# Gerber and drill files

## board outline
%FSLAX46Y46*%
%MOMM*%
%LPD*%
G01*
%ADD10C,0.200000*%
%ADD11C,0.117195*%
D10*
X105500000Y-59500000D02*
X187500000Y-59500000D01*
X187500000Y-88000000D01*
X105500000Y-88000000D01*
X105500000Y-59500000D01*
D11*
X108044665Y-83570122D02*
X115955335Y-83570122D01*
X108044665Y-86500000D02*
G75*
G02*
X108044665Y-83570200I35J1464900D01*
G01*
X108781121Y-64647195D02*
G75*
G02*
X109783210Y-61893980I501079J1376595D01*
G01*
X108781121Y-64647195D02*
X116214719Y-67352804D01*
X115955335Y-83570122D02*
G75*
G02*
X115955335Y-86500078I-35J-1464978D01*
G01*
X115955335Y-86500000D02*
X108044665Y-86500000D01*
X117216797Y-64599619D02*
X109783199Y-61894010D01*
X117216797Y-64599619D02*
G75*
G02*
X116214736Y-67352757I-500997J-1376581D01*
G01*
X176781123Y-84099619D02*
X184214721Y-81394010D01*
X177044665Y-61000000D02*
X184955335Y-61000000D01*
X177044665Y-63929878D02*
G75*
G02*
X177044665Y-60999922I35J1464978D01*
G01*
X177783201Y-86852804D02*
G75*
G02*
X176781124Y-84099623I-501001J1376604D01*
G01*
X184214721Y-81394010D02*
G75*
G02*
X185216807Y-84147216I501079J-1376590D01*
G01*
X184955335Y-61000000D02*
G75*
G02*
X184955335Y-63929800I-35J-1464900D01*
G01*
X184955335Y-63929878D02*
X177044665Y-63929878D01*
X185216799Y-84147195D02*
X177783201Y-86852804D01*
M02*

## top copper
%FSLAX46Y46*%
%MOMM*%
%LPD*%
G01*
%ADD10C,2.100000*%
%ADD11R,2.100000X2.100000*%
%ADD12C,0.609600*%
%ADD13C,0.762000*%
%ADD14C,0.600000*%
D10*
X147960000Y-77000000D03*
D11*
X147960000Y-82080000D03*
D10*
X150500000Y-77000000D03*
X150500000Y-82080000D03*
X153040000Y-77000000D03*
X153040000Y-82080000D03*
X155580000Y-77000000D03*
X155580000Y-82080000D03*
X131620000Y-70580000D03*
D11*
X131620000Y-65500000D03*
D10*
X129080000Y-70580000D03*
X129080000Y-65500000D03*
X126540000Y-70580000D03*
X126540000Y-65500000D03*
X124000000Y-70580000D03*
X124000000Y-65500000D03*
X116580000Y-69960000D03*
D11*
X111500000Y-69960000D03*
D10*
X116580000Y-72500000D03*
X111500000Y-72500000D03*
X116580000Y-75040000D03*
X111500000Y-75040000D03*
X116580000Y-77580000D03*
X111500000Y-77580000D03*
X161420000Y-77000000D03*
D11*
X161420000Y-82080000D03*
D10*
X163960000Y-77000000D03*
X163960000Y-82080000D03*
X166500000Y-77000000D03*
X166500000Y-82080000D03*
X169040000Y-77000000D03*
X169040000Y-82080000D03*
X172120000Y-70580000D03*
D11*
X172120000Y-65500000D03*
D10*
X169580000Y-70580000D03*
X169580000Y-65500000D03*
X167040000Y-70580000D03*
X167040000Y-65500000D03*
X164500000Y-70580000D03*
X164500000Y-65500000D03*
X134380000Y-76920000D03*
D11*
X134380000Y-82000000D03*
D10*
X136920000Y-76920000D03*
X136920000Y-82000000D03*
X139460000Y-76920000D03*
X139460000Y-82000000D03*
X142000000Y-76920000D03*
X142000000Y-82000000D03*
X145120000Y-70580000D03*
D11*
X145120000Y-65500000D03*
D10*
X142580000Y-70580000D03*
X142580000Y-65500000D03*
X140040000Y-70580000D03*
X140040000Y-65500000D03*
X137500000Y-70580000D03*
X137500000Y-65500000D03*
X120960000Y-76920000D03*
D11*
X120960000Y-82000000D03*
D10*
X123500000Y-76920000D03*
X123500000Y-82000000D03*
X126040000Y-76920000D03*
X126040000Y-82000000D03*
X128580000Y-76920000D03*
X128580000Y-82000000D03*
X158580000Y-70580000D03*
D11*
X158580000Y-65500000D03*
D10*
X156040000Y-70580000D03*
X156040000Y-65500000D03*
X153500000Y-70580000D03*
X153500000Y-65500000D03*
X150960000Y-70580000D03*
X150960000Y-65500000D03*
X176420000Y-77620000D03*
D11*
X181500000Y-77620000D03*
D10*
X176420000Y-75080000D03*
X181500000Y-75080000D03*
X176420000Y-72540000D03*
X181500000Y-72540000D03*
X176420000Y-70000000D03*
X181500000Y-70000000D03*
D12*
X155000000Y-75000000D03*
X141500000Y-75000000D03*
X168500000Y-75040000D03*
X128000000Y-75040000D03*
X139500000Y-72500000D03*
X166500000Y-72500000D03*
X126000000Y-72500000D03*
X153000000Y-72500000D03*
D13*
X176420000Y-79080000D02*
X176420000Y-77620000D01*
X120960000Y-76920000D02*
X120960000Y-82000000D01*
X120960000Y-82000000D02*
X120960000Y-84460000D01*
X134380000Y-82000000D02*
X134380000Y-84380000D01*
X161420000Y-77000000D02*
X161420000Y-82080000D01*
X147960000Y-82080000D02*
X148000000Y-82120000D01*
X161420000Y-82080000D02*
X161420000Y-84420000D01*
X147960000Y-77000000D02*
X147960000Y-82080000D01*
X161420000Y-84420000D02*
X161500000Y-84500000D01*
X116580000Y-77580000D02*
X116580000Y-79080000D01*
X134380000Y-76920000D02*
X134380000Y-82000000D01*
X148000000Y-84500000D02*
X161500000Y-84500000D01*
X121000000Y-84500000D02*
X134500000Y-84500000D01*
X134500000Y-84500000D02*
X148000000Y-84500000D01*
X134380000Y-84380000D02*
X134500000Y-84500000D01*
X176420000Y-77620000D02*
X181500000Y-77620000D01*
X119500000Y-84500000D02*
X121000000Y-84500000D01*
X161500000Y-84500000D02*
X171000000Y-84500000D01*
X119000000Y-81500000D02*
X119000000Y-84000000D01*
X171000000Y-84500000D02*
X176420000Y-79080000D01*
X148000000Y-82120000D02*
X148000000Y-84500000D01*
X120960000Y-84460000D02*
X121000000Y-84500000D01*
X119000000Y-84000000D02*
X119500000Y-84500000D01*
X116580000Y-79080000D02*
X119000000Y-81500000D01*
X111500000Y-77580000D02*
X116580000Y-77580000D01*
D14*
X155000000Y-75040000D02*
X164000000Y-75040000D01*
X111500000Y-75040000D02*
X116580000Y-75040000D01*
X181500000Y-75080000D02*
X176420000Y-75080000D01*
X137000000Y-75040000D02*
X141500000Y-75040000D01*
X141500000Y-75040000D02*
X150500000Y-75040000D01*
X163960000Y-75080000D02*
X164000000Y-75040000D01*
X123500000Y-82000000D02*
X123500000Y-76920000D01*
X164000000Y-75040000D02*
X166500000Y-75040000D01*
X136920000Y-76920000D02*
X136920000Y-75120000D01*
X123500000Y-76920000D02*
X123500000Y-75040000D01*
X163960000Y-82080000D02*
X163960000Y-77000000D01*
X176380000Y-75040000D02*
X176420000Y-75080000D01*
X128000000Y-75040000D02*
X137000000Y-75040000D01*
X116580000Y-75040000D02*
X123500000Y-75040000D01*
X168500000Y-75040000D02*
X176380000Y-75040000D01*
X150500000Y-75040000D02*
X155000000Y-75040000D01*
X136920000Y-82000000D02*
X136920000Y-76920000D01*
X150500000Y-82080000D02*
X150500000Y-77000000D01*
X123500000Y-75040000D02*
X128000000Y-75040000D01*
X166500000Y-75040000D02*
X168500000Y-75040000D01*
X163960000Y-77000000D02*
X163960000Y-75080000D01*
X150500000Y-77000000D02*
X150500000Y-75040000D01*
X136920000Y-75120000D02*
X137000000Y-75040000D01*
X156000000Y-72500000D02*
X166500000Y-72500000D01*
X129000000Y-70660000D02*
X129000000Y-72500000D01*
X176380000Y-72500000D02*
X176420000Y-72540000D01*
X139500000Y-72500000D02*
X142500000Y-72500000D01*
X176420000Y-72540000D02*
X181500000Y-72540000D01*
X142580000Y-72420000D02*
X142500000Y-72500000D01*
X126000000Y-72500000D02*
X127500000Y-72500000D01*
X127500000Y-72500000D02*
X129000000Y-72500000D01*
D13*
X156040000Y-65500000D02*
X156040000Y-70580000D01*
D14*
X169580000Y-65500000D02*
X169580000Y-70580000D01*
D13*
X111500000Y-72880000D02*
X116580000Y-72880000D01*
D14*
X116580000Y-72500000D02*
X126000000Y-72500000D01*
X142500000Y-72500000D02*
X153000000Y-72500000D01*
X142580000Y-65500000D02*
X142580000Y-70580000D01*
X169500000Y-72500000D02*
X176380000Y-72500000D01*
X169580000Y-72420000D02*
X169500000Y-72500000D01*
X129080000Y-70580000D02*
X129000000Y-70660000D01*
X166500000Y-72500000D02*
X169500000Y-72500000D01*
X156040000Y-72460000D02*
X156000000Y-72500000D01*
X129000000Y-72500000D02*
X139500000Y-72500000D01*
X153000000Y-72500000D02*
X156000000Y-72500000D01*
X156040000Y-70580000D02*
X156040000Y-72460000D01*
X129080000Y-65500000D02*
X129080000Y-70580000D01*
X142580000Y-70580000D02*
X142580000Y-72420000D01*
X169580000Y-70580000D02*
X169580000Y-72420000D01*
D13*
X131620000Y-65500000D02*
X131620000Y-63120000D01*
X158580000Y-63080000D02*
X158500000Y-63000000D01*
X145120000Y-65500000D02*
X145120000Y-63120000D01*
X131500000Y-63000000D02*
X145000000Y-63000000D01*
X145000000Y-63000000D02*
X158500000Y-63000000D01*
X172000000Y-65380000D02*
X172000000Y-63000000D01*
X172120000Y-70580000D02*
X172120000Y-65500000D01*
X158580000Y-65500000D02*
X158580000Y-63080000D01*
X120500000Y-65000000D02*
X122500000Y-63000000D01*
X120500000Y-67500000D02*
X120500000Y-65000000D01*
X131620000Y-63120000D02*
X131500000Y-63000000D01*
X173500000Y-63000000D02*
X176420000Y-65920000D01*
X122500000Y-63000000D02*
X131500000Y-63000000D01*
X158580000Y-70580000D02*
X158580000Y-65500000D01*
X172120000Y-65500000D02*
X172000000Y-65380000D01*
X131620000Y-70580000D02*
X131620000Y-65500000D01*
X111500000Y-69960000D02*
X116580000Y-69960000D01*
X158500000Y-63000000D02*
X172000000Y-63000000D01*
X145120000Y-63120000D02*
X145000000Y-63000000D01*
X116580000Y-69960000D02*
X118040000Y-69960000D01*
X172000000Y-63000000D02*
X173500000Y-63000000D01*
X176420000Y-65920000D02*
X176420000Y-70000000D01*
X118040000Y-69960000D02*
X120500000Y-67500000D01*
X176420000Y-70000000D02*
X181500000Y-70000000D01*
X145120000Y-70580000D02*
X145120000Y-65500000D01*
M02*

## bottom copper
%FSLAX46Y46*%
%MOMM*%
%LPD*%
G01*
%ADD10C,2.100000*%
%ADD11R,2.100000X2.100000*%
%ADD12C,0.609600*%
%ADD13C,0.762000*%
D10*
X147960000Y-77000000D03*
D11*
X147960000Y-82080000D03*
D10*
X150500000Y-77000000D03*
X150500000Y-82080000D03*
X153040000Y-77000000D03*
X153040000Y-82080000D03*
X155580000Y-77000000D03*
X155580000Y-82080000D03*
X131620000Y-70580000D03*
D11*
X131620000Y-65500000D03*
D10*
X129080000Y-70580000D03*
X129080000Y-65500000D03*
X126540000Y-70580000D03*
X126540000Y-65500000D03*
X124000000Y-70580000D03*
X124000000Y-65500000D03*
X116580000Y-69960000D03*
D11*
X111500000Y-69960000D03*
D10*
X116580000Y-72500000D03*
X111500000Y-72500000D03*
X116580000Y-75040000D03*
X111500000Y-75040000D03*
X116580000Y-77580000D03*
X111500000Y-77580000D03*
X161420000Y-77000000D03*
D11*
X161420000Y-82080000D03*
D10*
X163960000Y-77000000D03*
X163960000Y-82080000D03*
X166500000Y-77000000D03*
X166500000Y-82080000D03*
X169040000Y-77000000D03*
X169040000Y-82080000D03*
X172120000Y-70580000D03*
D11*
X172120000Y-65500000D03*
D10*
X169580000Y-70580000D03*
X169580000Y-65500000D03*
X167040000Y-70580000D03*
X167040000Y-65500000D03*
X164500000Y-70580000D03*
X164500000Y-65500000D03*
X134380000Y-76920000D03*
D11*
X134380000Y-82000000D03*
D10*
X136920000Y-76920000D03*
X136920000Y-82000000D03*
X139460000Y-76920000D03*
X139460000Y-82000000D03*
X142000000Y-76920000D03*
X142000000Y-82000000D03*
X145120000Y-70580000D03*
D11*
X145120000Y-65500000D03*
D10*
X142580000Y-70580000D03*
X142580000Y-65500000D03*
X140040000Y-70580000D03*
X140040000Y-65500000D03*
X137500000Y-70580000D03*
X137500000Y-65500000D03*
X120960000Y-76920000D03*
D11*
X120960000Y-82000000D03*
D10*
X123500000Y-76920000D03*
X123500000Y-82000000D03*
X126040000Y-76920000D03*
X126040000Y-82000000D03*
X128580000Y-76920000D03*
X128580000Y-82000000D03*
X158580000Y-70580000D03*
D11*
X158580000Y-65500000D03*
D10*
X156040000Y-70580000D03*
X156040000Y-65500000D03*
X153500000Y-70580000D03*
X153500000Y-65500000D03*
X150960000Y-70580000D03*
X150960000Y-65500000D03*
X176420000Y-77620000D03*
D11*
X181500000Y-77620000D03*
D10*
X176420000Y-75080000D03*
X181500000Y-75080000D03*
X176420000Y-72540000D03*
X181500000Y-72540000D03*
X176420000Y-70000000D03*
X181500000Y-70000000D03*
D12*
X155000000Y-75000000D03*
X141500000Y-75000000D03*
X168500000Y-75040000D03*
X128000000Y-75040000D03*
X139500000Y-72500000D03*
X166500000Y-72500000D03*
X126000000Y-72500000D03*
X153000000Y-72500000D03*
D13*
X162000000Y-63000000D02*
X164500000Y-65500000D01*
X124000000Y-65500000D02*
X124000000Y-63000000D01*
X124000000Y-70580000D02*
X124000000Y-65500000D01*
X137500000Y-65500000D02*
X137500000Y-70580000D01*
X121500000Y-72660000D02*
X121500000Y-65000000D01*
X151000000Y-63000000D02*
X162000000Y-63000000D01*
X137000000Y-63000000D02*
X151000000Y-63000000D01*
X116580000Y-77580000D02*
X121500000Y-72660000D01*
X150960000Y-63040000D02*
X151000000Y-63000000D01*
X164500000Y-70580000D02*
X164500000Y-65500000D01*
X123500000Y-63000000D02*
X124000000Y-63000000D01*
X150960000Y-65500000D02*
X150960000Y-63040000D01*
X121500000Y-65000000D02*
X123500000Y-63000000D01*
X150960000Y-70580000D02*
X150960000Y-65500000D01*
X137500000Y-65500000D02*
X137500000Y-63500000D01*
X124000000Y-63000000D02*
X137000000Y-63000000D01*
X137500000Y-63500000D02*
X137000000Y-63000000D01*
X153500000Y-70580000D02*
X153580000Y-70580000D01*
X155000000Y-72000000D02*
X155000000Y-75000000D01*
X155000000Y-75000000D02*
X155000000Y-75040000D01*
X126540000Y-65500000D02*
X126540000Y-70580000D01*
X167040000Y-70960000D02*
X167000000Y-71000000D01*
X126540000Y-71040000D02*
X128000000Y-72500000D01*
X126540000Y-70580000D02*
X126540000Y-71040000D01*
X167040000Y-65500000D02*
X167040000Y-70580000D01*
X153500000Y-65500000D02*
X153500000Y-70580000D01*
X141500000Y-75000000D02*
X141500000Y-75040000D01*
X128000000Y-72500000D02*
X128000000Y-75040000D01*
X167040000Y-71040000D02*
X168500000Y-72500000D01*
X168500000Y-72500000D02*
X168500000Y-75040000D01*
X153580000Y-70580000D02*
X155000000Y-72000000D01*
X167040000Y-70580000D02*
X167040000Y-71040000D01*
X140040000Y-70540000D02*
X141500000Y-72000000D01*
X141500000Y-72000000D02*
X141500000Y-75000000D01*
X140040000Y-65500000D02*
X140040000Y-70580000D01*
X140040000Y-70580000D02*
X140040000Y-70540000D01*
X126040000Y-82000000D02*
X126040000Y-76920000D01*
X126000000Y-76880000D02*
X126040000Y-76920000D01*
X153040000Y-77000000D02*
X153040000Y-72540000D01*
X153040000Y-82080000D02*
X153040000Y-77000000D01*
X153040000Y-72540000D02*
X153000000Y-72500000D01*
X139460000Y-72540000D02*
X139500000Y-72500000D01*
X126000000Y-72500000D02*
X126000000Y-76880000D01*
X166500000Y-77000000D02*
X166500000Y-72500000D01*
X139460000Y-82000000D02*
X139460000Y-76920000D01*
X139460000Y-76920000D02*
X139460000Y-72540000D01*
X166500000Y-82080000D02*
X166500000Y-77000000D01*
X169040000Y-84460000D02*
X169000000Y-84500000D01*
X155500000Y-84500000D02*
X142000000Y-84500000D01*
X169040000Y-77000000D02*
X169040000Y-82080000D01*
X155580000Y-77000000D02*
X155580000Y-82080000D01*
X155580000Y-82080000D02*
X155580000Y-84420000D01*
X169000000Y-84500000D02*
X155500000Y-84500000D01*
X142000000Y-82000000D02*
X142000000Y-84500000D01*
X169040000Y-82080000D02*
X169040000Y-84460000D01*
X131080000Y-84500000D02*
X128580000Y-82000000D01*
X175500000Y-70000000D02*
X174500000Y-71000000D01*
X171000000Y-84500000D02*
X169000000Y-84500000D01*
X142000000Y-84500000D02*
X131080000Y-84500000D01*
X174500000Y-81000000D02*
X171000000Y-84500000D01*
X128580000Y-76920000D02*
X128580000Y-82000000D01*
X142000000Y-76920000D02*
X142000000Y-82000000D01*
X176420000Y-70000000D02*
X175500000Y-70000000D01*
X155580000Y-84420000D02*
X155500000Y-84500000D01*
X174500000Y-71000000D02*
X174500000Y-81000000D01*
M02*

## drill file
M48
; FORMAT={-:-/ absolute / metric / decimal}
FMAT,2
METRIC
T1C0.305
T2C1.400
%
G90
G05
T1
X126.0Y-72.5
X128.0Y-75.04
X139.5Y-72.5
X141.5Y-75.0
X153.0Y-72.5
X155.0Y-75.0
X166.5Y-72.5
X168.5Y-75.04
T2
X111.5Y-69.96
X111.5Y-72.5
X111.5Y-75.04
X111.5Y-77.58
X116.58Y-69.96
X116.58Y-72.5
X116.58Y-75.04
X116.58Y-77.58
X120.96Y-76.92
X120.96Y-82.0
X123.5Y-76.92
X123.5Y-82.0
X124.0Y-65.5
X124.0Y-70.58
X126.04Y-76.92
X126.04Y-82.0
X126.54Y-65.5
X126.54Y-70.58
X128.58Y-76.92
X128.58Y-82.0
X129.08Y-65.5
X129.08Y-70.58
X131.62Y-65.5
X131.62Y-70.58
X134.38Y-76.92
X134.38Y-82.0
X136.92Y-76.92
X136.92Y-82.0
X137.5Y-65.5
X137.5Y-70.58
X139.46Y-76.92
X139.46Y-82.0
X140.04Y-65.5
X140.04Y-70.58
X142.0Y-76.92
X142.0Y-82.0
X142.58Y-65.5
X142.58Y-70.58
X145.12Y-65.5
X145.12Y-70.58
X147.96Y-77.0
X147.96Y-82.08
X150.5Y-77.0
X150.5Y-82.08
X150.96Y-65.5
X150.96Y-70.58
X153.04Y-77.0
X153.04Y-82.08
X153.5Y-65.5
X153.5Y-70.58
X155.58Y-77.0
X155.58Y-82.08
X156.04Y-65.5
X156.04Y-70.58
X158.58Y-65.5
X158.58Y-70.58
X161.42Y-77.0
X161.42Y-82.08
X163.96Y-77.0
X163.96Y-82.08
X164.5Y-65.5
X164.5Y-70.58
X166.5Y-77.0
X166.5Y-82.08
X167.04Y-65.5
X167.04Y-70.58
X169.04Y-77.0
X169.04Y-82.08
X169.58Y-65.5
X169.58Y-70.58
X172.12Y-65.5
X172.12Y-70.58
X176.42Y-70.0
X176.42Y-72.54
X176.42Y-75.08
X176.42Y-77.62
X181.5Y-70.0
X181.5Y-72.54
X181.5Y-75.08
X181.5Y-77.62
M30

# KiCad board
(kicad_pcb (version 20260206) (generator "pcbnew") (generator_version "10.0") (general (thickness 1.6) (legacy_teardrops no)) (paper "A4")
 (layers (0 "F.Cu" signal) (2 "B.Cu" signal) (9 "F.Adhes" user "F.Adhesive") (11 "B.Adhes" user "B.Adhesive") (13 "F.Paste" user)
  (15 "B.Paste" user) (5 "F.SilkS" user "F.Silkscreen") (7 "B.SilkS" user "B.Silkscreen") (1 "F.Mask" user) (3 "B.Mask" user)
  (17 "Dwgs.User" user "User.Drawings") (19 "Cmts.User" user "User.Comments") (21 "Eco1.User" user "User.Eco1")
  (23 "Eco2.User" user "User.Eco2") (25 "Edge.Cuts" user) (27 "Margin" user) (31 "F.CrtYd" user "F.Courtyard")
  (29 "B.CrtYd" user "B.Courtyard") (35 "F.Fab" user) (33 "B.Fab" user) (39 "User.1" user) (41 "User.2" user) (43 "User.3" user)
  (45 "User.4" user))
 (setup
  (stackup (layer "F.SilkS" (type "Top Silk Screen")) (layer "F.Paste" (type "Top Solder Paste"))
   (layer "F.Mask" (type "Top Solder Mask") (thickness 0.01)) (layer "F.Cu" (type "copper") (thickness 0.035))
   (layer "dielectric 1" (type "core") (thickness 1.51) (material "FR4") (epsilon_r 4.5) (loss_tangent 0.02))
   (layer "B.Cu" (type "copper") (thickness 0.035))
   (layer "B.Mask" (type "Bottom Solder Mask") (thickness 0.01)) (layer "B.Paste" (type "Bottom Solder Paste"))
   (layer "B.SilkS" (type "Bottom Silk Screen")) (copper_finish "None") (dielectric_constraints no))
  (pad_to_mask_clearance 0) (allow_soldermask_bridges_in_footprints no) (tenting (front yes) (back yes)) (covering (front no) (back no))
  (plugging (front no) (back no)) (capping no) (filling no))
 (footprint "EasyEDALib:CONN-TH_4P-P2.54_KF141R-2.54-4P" (layer "F.Cu") (at 151.77 79.54)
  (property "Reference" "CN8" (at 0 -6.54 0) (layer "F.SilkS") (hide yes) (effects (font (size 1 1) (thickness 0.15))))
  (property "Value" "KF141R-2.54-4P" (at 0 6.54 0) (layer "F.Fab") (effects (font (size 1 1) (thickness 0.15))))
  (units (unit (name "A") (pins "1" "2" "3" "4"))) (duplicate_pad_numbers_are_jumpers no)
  (pad "1" thru_hole circle (at -3.81 -2.54 180) (size 2.1 2.1) (drill 1.399998) (layers "*.Cu" "*.Mask") (remove_unused_layers no)
   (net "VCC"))
  (pad "1" thru_hole rect (at -3.81 2.54 180) (size 2.1 2.1) (drill 1.399998) (layers "*.Cu" "*.Mask") (remove_unused_layers no) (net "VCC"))
  (pad "2" thru_hole circle (at -1.27 -2.54 180) (size 2.1 2.1) (drill 1.399998) (layers "*.Cu" "*.Mask") (remove_unused_layers no)
   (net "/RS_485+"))
  (pad "2" thru_hole circle (at -1.27 2.54 180) (size 2.1 2.1) (drill 1.399998) (layers "*.Cu" "*.Mask") (remove_unused_layers no)
   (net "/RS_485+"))
  (pad "3" thru_hole circle (at 1.27 -2.54 180) (size 2.1 2.1) (drill 1.399998) (layers "*.Cu" "*.Mask") (remove_unused_layers no)
   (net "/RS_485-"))
  (pad "3" thru_hole circle (at 1.27 2.54 180) (size 2.1 2.1) (drill 1.399998) (layers "*.Cu" "*.Mask") (remove_unused_layers no)
   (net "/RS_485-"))
  (pad "4" thru_hole circle (at 3.81 -2.54 180) (size 2.1 2.1) (drill 1.399998) (layers "*.Cu" "*.Mask") (remove_unused_layers no)
   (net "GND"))
  (pad "4" thru_hole circle (at 3.81 2.54 180) (size 2.1 2.1) (drill 1.399998) (layers "*.Cu" "*.Mask") (remove_unused_layers no)
   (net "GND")))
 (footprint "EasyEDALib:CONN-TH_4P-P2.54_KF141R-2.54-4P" (layer "F.Cu") (at 127.81 68.04 180)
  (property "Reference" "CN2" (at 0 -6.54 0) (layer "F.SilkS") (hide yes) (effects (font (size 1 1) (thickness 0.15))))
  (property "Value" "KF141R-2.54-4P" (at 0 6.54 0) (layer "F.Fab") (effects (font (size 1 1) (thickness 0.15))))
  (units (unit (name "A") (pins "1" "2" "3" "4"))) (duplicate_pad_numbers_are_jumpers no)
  (pad "1" thru_hole circle (at -3.81 -2.54) (size 2.1 2.1) (drill 1.399998) (layers "*.Cu" "*.Mask") (remove_unused_layers no) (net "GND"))
  (pad "1" thru_hole rect (at -3.81 2.54) (size 2.1 2.1) (drill 1.399998) (layers "*.Cu" "*.Mask") (remove_unused_layers no) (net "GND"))
  (pad "2" thru_hole circle (at -1.27 -2.54) (size 2.1 2.1) (drill 1.399998) (layers "*.Cu" "*.Mask") (remove_unused_layers no)
   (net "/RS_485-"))
  (pad "2" thru_hole circle (at -1.27 2.54) (size 2.1 2.1) (drill 1.399998) (layers "*.Cu" "*.Mask") (remove_unused_layers no)
   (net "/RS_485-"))
  (pad "3" thru_hole circle (at 1.27 -2.54) (size 2.1 2.1) (drill 1.399998) (layers "*.Cu" "*.Mask") (remove_unused_layers no)
   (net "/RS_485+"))
  (pad "3" thru_hole circle (at 1.27 2.54) (size 2.1 2.1) (drill 1.399998) (layers "*.Cu" "*.Mask") (remove_unused_layers no)
   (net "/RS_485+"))
  (pad "4" thru_hole circle (at 3.81 -2.54) (size 2.1 2.1) (drill 1.399998) (layers "*.Cu" "*.Mask") (remove_unused_layers no) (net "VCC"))
  (pad "4" thru_hole circle (at 3.81 2.54) (size 2.1 2.1) (drill 1.399998) (layers "*.Cu" "*.Mask") (remove_unused_layers no) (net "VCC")))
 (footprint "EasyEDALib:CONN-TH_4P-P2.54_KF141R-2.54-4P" (layer "F.Cu") (at 114.04 73.77 -90)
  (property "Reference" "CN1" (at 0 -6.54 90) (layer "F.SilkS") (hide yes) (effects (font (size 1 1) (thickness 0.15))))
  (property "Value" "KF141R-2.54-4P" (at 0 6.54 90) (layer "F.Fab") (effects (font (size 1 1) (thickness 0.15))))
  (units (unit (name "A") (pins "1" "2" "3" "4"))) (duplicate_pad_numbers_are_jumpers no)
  (pad "1" thru_hole circle (at -3.81 -2.54 90) (size 2.1 2.1) (drill 1.399998) (layers "*.Cu" "*.Mask") (remove_unused_layers no)
   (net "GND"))
  (pad "1" thru_hole rect (at -3.81 2.54 90) (size 2.1 2.1) (drill 1.399998) (layers "*.Cu" "*.Mask") (remove_unused_layers no) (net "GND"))
  (pad "2" thru_hole circle (at -1.27 -2.54 90) (size 2.1 2.1) (drill 1.399998) (layers "*.Cu" "*.Mask") (remove_unused_layers no)
   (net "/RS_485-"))
  (pad "2" thru_hole circle (at -1.27 2.54 90) (size 2.1 2.1) (drill 1.399998) (layers "*.Cu" "*.Mask") (remove_unused_layers no)
   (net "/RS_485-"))
  (pad "3" thru_hole circle (at 1.27 -2.54 90) (size 2.1 2.1) (drill 1.399998) (layers "*.Cu" "*.Mask") (remove_unused_layers no)
   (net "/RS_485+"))
  (pad "3" thru_hole circle (at 1.27 2.54 90) (size 2.1 2.1) (drill 1.399998) (layers "*.Cu" "*.Mask") (remove_unused_layers no)
   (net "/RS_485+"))
  (pad "4" thru_hole circle (at 3.81 -2.54 90) (size 2.1 2.1) (drill 1.399998) (layers "*.Cu" "*.Mask") (remove_unused_layers no)
   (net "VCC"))
  (pad "4" thru_hole circle (at 3.81 2.54 90) (size 2.1 2.1) (drill 1.399998) (layers "*.Cu" "*.Mask") (remove_unused_layers no) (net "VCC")))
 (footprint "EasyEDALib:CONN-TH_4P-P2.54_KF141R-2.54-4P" (layer "F.Cu") (at 165.23 79.54)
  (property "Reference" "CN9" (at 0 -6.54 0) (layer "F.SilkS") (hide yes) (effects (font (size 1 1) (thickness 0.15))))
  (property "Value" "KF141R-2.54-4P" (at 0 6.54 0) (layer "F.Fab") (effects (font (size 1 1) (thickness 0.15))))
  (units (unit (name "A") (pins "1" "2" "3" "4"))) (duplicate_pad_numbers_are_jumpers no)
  (pad "1" thru_hole circle (at -3.81 -2.54 180) (size 2.1 2.1) (drill 1.399998) (layers "*.Cu" "*.Mask") (remove_unused_layers no)
   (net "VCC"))
  (pad "1" thru_hole rect (at -3.81 2.54 180) (size 2.1 2.1) (drill 1.399998) (layers "*.Cu" "*.Mask") (remove_unused_layers no) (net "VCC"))
  (pad "2" thru_hole circle (at -1.27 -2.54 180) (size 2.1 2.1) (drill 1.399998) (layers "*.Cu" "*.Mask") (remove_unused_layers no)
   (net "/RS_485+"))
  (pad "2" thru_hole circle (at -1.27 2.54 180) (size 2.1 2.1) (drill 1.399998) (layers "*.Cu" "*.Mask") (remove_unused_layers no)
   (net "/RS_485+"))
  (pad "3" thru_hole circle (at 1.27 -2.54 180) (size 2.1 2.1) (drill 1.399998) (layers "*.Cu" "*.Mask") (remove_unused_layers no)
   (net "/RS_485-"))
  (pad "3" thru_hole circle (at 1.27 2.54 180) (size 2.1 2.1) (drill 1.399998) (layers "*.Cu" "*.Mask") (remove_unused_layers no)
   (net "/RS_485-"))
  (pad "4" thru_hole circle (at 3.81 -2.54 180) (size 2.1 2.1) (drill 1.399998) (layers "*.Cu" "*.Mask") (remove_unused_layers no)
   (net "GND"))
  (pad "4" thru_hole circle (at 3.81 2.54 180) (size 2.1 2.1) (drill 1.399998) (layers "*.Cu" "*.Mask") (remove_unused_layers no)
   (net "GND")))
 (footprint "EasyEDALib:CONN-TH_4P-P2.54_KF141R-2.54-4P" (layer "F.Cu") (at 168.31 68.04 180)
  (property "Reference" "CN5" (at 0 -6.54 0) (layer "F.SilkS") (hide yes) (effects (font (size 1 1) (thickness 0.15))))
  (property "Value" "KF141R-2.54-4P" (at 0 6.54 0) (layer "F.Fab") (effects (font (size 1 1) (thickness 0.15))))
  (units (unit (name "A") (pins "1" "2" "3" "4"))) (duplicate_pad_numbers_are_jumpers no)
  (pad "1" thru_hole circle (at -3.81 -2.54) (size 2.1 2.1) (drill 1.399998) (layers "*.Cu" "*.Mask") (remove_unused_layers no) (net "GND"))
  (pad "1" thru_hole rect (at -3.81 2.54) (size 2.1 2.1) (drill 1.399998) (layers "*.Cu" "*.Mask") (remove_unused_layers no) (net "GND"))
  (pad "2" thru_hole circle (at -1.27 -2.54) (size 2.1 2.1) (drill 1.399998) (layers "*.Cu" "*.Mask") (remove_unused_layers no)
   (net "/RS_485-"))
  (pad "2" thru_hole circle (at -1.27 2.54) (size 2.1 2.1) (drill 1.399998) (layers "*.Cu" "*.Mask") (remove_unused_layers no)
   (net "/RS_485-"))
  (pad "3" thru_hole circle (at 1.27 -2.54) (size 2.1 2.1) (drill 1.399998) (layers "*.Cu" "*.Mask") (remove_unused_layers no)
   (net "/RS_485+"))
  (pad "3" thru_hole circle (at 1.27 2.54) (size 2.1 2.1) (drill 1.399998) (layers "*.Cu" "*.Mask") (remove_unused_layers no)
   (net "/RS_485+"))
  (pad "4" thru_hole circle (at 3.81 -2.54) (size 2.1 2.1) (drill 1.399998) (layers "*.Cu" "*.Mask") (remove_unused_layers no) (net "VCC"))
  (pad "4" thru_hole circle (at 3.81 2.54) (size 2.1 2.1) (drill 1.399998) (layers "*.Cu" "*.Mask") (remove_unused_layers no) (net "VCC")))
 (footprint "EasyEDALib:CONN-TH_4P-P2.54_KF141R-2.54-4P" (layer "F.Cu") (at 138.19 79.46)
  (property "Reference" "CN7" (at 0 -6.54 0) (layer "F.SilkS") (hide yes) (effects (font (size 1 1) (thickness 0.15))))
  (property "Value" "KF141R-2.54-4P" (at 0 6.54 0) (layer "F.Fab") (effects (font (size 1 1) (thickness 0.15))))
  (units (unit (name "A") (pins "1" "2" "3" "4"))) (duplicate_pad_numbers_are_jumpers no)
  (pad "1" thru_hole circle (at -3.81 -2.54 180) (size 2.1 2.1) (drill 1.399998) (layers "*.Cu" "*.Mask") (remove_unused_layers no)
   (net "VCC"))
  (pad "1" thru_hole rect (at -3.81 2.54 180) (size 2.1 2.1) (drill 1.399998) (layers "*.Cu" "*.Mask") (remove_unused_layers no) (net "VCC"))
  (pad "2" thru_hole circle (at -1.27 -2.54 180) (size 2.1 2.1) (drill 1.399998) (layers "*.Cu" "*.Mask") (remove_unused_layers no)
   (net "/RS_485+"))
  (pad "2" thru_hole circle (at -1.27 2.54 180) (size 2.1 2.1) (drill 1.399998) (layers "*.Cu" "*.Mask") (remove_unused_layers no)
   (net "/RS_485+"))
  (pad "3" thru_hole circle (at 1.27 -2.54 180) (size 2.1 2.1) (drill 1.399998) (layers "*.Cu" "*.Mask") (remove_unused_layers no)
   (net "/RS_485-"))
  (pad "3" thru_hole circle (at 1.27 2.54 180) (size 2.1 2.1) (drill 1.399998) (layers "*.Cu" "*.Mask") (remove_unused_layers no)
   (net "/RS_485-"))
  (pad "4" thru_hole circle (at 3.81 -2.54 180) (size 2.1 2.1) (drill 1.399998) (layers "*.Cu" "*.Mask") (remove_unused_layers no)
   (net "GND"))
  (pad "4" thru_hole circle (at 3.81 2.54 180) (size 2.1 2.1) (drill 1.399998) (layers "*.Cu" "*.Mask") (remove_unused_layers no)
   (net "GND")))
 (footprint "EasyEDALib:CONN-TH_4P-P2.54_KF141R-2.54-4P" (layer "F.Cu") (at 141.31 68.04 180)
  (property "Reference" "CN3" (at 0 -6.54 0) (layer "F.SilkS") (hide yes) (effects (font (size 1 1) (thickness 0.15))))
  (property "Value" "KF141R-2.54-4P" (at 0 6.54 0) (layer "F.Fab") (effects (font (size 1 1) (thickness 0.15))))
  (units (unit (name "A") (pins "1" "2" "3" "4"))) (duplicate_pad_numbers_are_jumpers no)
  (pad "1" thru_hole circle (at -3.81 -2.54) (size 2.1 2.1) (drill 1.399998) (layers "*.Cu" "*.Mask") (remove_unused_layers no) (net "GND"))
  (pad "1" thru_hole rect (at -3.81 2.54) (size 2.1 2.1) (drill 1.399998) (layers "*.Cu" "*.Mask") (remove_unused_layers no) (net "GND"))
  (pad "2" thru_hole circle (at -1.27 -2.54) (size 2.1 2.1) (drill 1.399998) (layers "*.Cu" "*.Mask") (remove_unused_layers no)
   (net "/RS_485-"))
  (pad "2" thru_hole circle (at -1.27 2.54) (size 2.1 2.1) (drill 1.399998) (layers "*.Cu" "*.Mask") (remove_unused_layers no)
   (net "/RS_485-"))
  (pad "3" thru_hole circle (at 1.27 -2.54) (size 2.1 2.1) (drill 1.399998) (layers "*.Cu" "*.Mask") (remove_unused_layers no)
   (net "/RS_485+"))
  (pad "3" thru_hole circle (at 1.27 2.54) (size 2.1 2.1) (drill 1.399998) (layers "*.Cu" "*.Mask") (remove_unused_layers no)
   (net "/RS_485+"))
  (pad "4" thru_hole circle (at 3.81 -2.54) (size 2.1 2.1) (drill 1.399998) (layers "*.Cu" "*.Mask") (remove_unused_layers no) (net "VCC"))
  (pad "4" thru_hole circle (at 3.81 2.54) (size 2.1 2.1) (drill 1.399998) (layers "*.Cu" "*.Mask") (remove_unused_layers no) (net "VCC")))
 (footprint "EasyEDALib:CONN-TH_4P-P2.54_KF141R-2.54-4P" (layer "F.Cu") (at 124.77 79.46)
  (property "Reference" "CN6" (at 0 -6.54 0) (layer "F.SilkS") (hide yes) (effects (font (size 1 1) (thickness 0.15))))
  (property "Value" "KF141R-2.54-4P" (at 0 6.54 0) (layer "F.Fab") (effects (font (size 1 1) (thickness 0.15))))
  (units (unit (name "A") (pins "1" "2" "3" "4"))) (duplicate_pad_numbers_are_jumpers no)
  (pad "1" thru_hole circle (at -3.81 -2.54 180) (size 2.1 2.1) (drill 1.399998) (layers "*.Cu" "*.Mask") (remove_unused_layers no)
   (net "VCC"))
  (pad "1" thru_hole rect (at -3.81 2.54 180) (size 2.1 2.1) (drill 1.399998) (layers "*.Cu" "*.Mask") (remove_unused_layers no) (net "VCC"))
  (pad "2" thru_hole circle (at -1.27 -2.54 180) (size 2.1 2.1) (drill 1.399998) (layers "*.Cu" "*.Mask") (remove_unused_layers no)
   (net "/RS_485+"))
  (pad "2" thru_hole circle (at -1.27 2.54 180) (size 2.1 2.1) (drill 1.399998) (layers "*.Cu" "*.Mask") (remove_unused_layers no)
   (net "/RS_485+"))
  (pad "3" thru_hole circle (at 1.27 -2.54 180) (size 2.1 2.1) (drill 1.399998) (layers "*.Cu" "*.Mask") (remove_unused_layers no)
   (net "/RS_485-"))
  (pad "3" thru_hole circle (at 1.27 2.54 180) (size 2.1 2.1) (drill 1.399998) (layers "*.Cu" "*.Mask") (remove_unused_layers no)
   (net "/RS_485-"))
  (pad "4" thru_hole circle (at 3.81 -2.54 180) (size 2.1 2.1) (drill 1.399998) (layers "*.Cu" "*.Mask") (remove_unused_layers no)
   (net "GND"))
  (pad "4" thru_hole circle (at 3.81 2.54 180) (size 2.1 2.1) (drill 1.399998) (layers "*.Cu" "*.Mask") (remove_unused_layers no)
   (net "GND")))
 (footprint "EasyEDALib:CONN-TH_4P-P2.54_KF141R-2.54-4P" (layer "F.Cu") (at 154.77 68.04 180)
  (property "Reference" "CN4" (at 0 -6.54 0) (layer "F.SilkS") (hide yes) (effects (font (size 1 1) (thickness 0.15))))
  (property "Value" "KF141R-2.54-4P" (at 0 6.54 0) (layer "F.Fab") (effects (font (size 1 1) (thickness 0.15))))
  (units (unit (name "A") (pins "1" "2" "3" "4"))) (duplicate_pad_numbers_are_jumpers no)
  (pad "1" thru_hole circle (at -3.81 -2.54) (size 2.1 2.1) (drill 1.399998) (layers "*.Cu" "*.Mask") (remove_unused_layers no) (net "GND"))
  (pad "1" thru_hole rect (at -3.81 2.54) (size 2.1 2.1) (drill 1.399998) (layers "*.Cu" "*.Mask") (remove_unused_layers no) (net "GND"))
  (pad "2" thru_hole circle (at -1.27 -2.54) (size 2.1 2.1) (drill 1.399998) (layers "*.Cu" "*.Mask") (remove_unused_layers no)
   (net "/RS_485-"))
  (pad "2" thru_hole circle (at -1.27 2.54) (size 2.1 2.1) (drill 1.399998) (layers "*.Cu" "*.Mask") (remove_unused_layers no)
   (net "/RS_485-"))
  (pad "3" thru_hole circle (at 1.27 -2.54) (size 2.1 2.1) (drill 1.399998) (layers "*.Cu" "*.Mask") (remove_unused_layers no)
   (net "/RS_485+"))
  (pad "3" thru_hole circle (at 1.27 2.54) (size 2.1 2.1) (drill 1.399998) (layers "*.Cu" "*.Mask") (remove_unused_layers no)
   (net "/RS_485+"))
  (pad "4" thru_hole circle (at 3.81 -2.54) (size 2.1 2.1) (drill 1.399998) (layers "*.Cu" "*.Mask") (remove_unused_layers no) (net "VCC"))
  (pad "4" thru_hole circle (at 3.81 2.54) (size 2.1 2.1) (drill 1.399998) (layers "*.Cu" "*.Mask") (remove_unused_layers no) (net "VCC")))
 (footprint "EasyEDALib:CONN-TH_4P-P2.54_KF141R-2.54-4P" (layer "F.Cu") (at 178.96 73.81 90)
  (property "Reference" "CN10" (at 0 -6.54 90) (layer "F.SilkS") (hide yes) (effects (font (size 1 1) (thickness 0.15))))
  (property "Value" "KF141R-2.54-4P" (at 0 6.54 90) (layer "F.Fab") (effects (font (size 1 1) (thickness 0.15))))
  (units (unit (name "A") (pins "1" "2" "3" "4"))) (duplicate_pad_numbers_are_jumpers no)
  (pad "1" thru_hole circle (at -3.81 -2.54 270) (size 2.1 2.1) (drill 1.399998) (layers "*.Cu" "*.Mask") (remove_unused_layers no)
   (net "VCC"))
  (pad "1" thru_hole rect (at -3.81 2.54 270) (size 2.1 2.1) (drill 1.399998) (layers "*.Cu" "*.Mask") (remove_unused_layers no) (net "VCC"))
  (pad "2" thru_hole circle (at -1.27 -2.54 270) (size 2.1 2.1) (drill 1.399998) (layers "*.Cu" "*.Mask") (remove_unused_layers no)
   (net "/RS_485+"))
  (pad "2" thru_hole circle (at -1.27 2.54 270) (size 2.1 2.1) (drill 1.399998) (layers "*.Cu" "*.Mask") (remove_unused_layers no)
   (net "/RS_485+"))
  (pad "3" thru_hole circle (at 1.27 -2.54 270) (size 2.1 2.1) (drill 1.399998) (layers "*.Cu" "*.Mask") (remove_unused_layers no)
   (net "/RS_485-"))
  (pad "3" thru_hole circle (at 1.27 2.54 270) (size 2.1 2.1) (drill 1.399998) (layers "*.Cu" "*.Mask") (remove_unused_layers no)
   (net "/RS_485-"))
  (pad "4" thru_hole circle (at 3.81 -2.54 270) (size 2.1 2.1) (drill 1.399998) (layers "*.Cu" "*.Mask") (remove_unused_layers no)
   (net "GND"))
  (pad "4" thru_hole circle (at 3.81 2.54 270) (size 2.1 2.1) (drill 1.399998) (layers "*.Cu" "*.Mask") (remove_unused_layers no)
   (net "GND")))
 (gr_rect (start 105.5 59.5) (end 187.5 88) (stroke (width 0.2) (type solid)) (fill no) (layer "Edge.Cuts"))
 (gr_line (start 108.044665 83.570122) (end 115.955335 83.570122) (stroke (width 0.117195) (type default)) (layer "Edge.Cuts"))
 (gr_arc (start 108.044665 86.5) (mid 106.579726 85.035061) (end 108.044665 83.570122) (stroke (width 0.117195) (type default))
  (layer "Edge.Cuts"))
 (gr_arc (start 108.781121 64.647195) (mid 107.905565 62.76956) (end 109.783199 61.89401) (stroke (width 0.117195) (type default))
  (layer "Edge.Cuts"))
 (gr_line (start 108.781121 64.647195) (end 116.214719 67.352804) (stroke (width 0.117195) (type default)) (layer "Edge.Cuts"))
 (gr_arc (start 115.955335 83.570122) (mid 117.420274 85.035061) (end 115.955335 86.5) (stroke (width 0.117195) (type default))
  (layer "Edge.Cuts"))
 (gr_line (start 115.955335 86.5) (end 108.044665 86.5) (stroke (width 0.117195) (type default)) (layer "Edge.Cuts"))
 (gr_line (start 117.216797 64.599619) (end 109.783199 61.89401) (stroke (width 0.117195) (type default)) (layer "Edge.Cuts"))
 (gr_arc (start 117.216797 64.599619) (mid 118.092351 66.477251) (end 116.214719 67.352804) (stroke (width 0.117195) (type default))
  (layer "Edge.Cuts"))
 (gr_line (start 176.781123 84.099619) (end 184.214721 81.39401) (stroke (width 0.117195) (type default)) (layer "Edge.Cuts"))
 (gr_line (start 177.044665 61) (end 184.955335 61) (stroke (width 0.117195) (type default)) (layer "Edge.Cuts"))
 (gr_arc (start 177.044665 63.929878) (mid 175.579726 62.464939) (end 177.044665 61) (stroke (width 0.117195) (type default))
  (layer "Edge.Cuts"))
 (gr_arc (start 177.783201 86.852804) (mid 175.905569 85.97725) (end 176.781123 84.099619) (stroke (width 0.117195) (type default))
  (layer "Edge.Cuts"))
 (gr_arc (start 184.214721 81.39401) (mid 186.092353 82.269564) (end 185.216799 84.147195) (stroke (width 0.117195) (type default))
  (layer "Edge.Cuts"))
 (gr_arc (start 184.955335 61) (mid 186.420274 62.464939) (end 184.955335 63.929878) (stroke (width 0.117195) (type default))
  (layer "Edge.Cuts"))
 (gr_line (start 184.955335 63.929878) (end 177.044665 63.929878) (stroke (width 0.117195) (type default)) (layer "Edge.Cuts"))
 (gr_line (start 185.216799 84.147195) (end 177.783201 86.852804) (stroke (width 0.117195) (type default)) (layer "Edge.Cuts"))
 (segment (start 176.42 79.08) (end 176.42 77.62) (width 0.762) (layer "F.Cu") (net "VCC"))
 (segment (start 120.96 76.92) (end 120.96 82) (width 0.762) (layer "F.Cu") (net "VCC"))
 (segment (start 120.96 82) (end 120.96 84.46) (width 0.762) (layer "F.Cu") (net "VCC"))
 (segment (start 134.38 82) (end 134.38 84.38) (width 0.762) (layer "F.Cu") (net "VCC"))
 (segment (start 161.42 77) (end 161.42 82.08) (width 0.762) (layer "F.Cu") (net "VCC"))
 (segment (start 147.96 82.08) (end 148 82.12) (width 0.762) (layer "F.Cu") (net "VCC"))
 (segment (start 161.42 82.08) (end 161.42 84.42) (width 0.762) (layer "F.Cu") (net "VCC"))
 (segment (start 147.96 77) (end 147.96 82.08) (width 0.762) (layer "F.Cu") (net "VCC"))
 (segment (start 161.42 84.42) (end 161.5 84.5) (width 0.762) (layer "F.Cu") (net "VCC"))
 (segment (start 116.58 77.58) (end 116.58 79.08) (width 0.762) (layer "F.Cu") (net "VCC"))
 (segment (start 134.38 76.92) (end 134.38 82) (width 0.762) (layer "F.Cu") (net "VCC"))
 (segment (start 148 84.5) (end 161.5 84.5) (width 0.762) (layer "F.Cu") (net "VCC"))
 (segment (start 121 84.5) (end 134.5 84.5) (width 0.762) (layer "F.Cu") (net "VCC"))
 (segment (start 134.5 84.5) (end 148 84.5) (width 0.762) (layer "F.Cu") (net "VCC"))
 (segment (start 134.38 84.38) (end 134.5 84.5) (width 0.762) (layer "F.Cu") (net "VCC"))
 (segment (start 176.42 77.62) (end 181.5 77.62) (width 0.762) (layer "F.Cu") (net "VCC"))
 (segment (start 119.5 84.5) (end 121 84.5) (width 0.762) (layer "F.Cu") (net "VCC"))
 (segment (start 161.5 84.5) (end 171 84.5) (width 0.762) (layer "F.Cu") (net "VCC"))
 (segment (start 119 81.5) (end 119 84) (width 0.762) (layer "F.Cu") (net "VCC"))
 (segment (start 171 84.5) (end 176.42 79.08) (width 0.762) (layer "F.Cu") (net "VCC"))
 (segment (start 148 82.12) (end 148 84.5) (width 0.762) (layer "F.Cu") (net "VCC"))
 (segment (start 120.96 84.46) (end 121 84.5) (width 0.762) (layer "F.Cu") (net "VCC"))
 (segment (start 119 84) (end 119.5 84.5) (width 0.762) (layer "F.Cu") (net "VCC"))
 (segment (start 116.58 79.08) (end 119 81.5) (width 0.762) (layer "F.Cu") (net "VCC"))
 (segment (start 111.5 77.58) (end 116.58 77.58) (width 0.762) (layer "F.Cu") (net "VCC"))
 (segment (start 162 63) (end 164.5 65.5) (width 0.762) (layer "B.Cu") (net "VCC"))
 (segment (start 124 65.5) (end 124 63) (width 0.762) (layer "B.Cu") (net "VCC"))
 (segment (start 124 70.58) (end 124 65.5) (width 0.762) (layer "B.Cu") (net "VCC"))
 (segment (start 137.5 65.5) (end 137.5 70.58) (width 0.762) (layer "B.Cu") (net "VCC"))
 (segment (start 121.5 72.66) (end 121.5 65) (width 0.762) (layer "B.Cu") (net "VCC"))
 (segment (start 151 63) (end 162 63) (width 0.762) (layer "B.Cu") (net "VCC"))
 (segment (start 137 63) (end 151 63) (width 0.762) (layer "B.Cu") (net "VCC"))
 (segment (start 116.58 77.58) (end 121.5 72.66) (width 0.762) (layer "B.Cu") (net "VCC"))
 (segment (start 150.96 63.04) (end 151 63) (width 0.762) (layer "B.Cu") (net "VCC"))
 (segment (start 164.5 70.58) (end 164.5 65.5) (width 0.762) (layer "B.Cu") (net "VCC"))
 (segment (start 123.5 63) (end 124 63) (width 0.762) (layer "B.Cu") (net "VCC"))
 (segment (start 150.96 65.5) (end 150.96 63.04) (width 0.762) (layer "B.Cu") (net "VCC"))
 (segment (start 121.5 65) (end 123.5 63) (width 0.762) (layer "B.Cu") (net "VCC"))
 (segment (start 150.96 70.58) (end 150.96 65.5) (width 0.762) (layer "B.Cu") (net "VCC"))
 (segment (start 137.5 65.5) (end 137.5 63.5) (width 0.762) (layer "B.Cu") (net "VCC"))
 (segment (start 124 63) (end 137 63) (width 0.762) (layer "B.Cu") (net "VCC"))
 (segment (start 137.5 63.5) (end 137 63) (width 0.762) (layer "B.Cu") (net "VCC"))
 (segment (start 155 75.04) (end 164 75.04) (width 0.6) (layer "F.Cu") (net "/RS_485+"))
 (segment (start 111.5 75.04) (end 116.58 75.04) (width 0.6) (layer "F.Cu") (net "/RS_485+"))
 (segment (start 181.5 75.08) (end 176.42 75.08) (width 0.6) (layer "F.Cu") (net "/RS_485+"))
 (segment (start 137 75.04) (end 141.5 75.04) (width 0.6) (layer "F.Cu") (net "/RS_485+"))
 (segment (start 141.5 75.04) (end 150.5 75.04) (width 0.6) (layer "F.Cu") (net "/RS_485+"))
 (segment (start 163.96 75.08) (end 164 75.04) (width 0.6) (layer "F.Cu") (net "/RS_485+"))
 (segment (start 123.5 82) (end 123.5 76.92) (width 0.6) (layer "F.Cu") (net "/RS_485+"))
 (segment (start 164 75.04) (end 166.5 75.04) (width 0.6) (layer "F.Cu") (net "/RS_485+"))
 (segment (start 136.92 76.92) (end 136.92 75.12) (width 0.6) (layer "F.Cu") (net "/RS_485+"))
 (segment (start 123.5 76.92) (end 123.5 75.04) (width 0.6) (layer "F.Cu") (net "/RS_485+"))
 (segment (start 163.96 82.08) (end 163.96 77) (width 0.6) (layer "F.Cu") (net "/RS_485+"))
 (segment (start 176.38 75.04) (end 176.42 75.08) (width 0.6) (layer "F.Cu") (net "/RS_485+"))
 (segment (start 128 75.04) (end 137 75.04) (width 0.6) (layer "F.Cu") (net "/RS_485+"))
 (segment (start 116.58 75.04) (end 123.5 75.04) (width 0.6) (layer "F.Cu") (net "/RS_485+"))
 (segment (start 168.5 75.04) (end 176.38 75.04) (width 0.6) (layer "F.Cu") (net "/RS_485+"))
 (segment (start 150.5 75.04) (end 155 75.04) (width 0.6) (layer "F.Cu") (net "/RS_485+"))
 (segment (start 136.92 82) (end 136.92 76.92) (width 0.6) (layer "F.Cu") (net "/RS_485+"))
 (segment (start 150.5 82.08) (end 150.5 77) (width 0.6) (layer "F.Cu") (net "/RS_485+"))
 (segment (start 123.5 75.04) (end 128 75.04) (width 0.6) (layer "F.Cu") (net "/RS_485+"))
 (segment (start 166.5 75.04) (end 168.5 75.04) (width 0.6) (layer "F.Cu") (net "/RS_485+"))
 (segment (start 163.96 77) (end 163.96 75.08) (width 0.6) (layer "F.Cu") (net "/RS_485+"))
 (segment (start 150.5 77) (end 150.5 75.04) (width 0.6) (layer "F.Cu") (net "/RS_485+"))
 (segment (start 136.92 75.12) (end 137 75.04) (width 0.6) (layer "F.Cu") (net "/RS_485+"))
 (via (at 155 75) (size 0.6096) (drill 0.3048) (layers "F.Cu" "B.Cu") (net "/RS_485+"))
 (via (at 141.5 75) (size 0.6096) (drill 0.3048) (layers "F.Cu" "B.Cu") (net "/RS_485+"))
 (via (at 168.5 75.04) (size 0.6096) (drill 0.3048) (layers "F.Cu" "B.Cu") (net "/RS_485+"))
 (via (at 128 75.04) (size 0.6096) (drill 0.3048) (layers "F.Cu" "B.Cu") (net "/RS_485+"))
 (segment (start 153.5 70.58) (end 153.58 70.58) (width 0.762) (layer "B.Cu") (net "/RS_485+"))
 (segment (start 155 72) (end 155 75) (width 0.762) (layer "B.Cu") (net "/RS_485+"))
 (segment (start 155 75) (end 155 75.04) (width 0.762) (layer "B.Cu") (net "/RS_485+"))
 (segment (start 126.54 65.5) (end 126.54 70.58) (width 0.762) (layer "B.Cu") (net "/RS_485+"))
 (segment (start 167.04 70.96) (end 167 71) (width 0.762) (layer "B.Cu") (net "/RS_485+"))
 (segment (start 126.54 71.04) (end 128 72.5) (width 0.762) (layer "B.Cu") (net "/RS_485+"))
 (segment (start 126.54 70.58) (end 126.54 71.04) (width 0.762) (layer "B.Cu") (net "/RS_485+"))
 (segment (start 167.04 65.5) (end 167.04 70.58) (width 0.762) (layer "B.Cu") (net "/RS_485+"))
 (segment (start 153.5 65.5) (end 153.5 70.58) (width 0.762) (layer "B.Cu") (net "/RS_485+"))
 (segment (start 141.5 75) (end 141.5 75.04) (width 0.762) (layer "B.Cu") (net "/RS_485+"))
 (segment (start 128 72.5) (end 128 75.04) (width 0.762) (layer "B.Cu") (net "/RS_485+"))
 (segment (start 167.04 71.04) (end 168.5 72.5) (width 0.762) (layer "B.Cu") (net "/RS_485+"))
 (segment (start 168.5 72.5) (end 168.5 75.04) (width 0.762) (layer "B.Cu") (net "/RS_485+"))
 (segment (start 153.58 70.58) (end 155 72) (width 0.762) (layer "B.Cu") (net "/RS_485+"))
 (segment (start 167.04 70.58) (end 167.04 71.04) (width 0.762) (layer "B.Cu") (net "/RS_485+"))
 (segment (start 140.04 70.54) (end 141.5 72) (width 0.762) (layer "B.Cu") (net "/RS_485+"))
 (segment (start 141.5 72) (end 141.5 75) (width 0.762) (layer "B.Cu") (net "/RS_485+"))
 (segment (start 140.04 65.5) (end 140.04 70.58) (width 0.762) (layer "B.Cu") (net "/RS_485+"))
 (segment (start 140.04 70.58) (end 140.04 70.54) (width 0.762) (layer "B.Cu") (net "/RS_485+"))
 (segment (start 156 72.5) (end 166.5 72.5) (width 0.6) (layer "F.Cu") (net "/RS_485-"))
 (segment (start 129 70.66) (end 129 72.5) (width 0.6) (layer "F.Cu") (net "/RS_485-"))
 (segment (start 176.38 72.5) (end 176.42 72.54) (width 0.6) (layer "F.Cu") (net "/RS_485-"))
 (segment (start 139.5 72.5) (end 142.5 72.5) (width 0.6) (layer "F.Cu") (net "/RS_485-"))
 (segment (start 176.42 72.54) (end 181.5 72.54) (width 0.6) (layer "F.Cu") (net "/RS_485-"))
 (segment (start 142.58 72.42) (end 142.5 72.5) (width 0.6) (layer "F.Cu") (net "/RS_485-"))
 (segment (start 126 72.5) (end 127.5 72.5) (width 0.6) (layer "F.Cu") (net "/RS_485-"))
 (segment (start 127.5 72.5) (end 129 72.5) (width 0.6) (layer "F.Cu") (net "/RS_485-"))
 (segment (start 156.04 65.5) (end 156.04 70.58) (width 0.762) (layer "F.Cu") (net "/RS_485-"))
 (segment (start 169.58 65.5) (end 169.58 70.58) (width 0.6) (layer "F.Cu") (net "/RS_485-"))
 (segment (start 111.5 72.88) (end 116.58 72.88) (width 0.762) (layer "F.Cu") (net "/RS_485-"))
 (segment (start 116.58 72.5) (end 126 72.5) (width 0.6) (layer "F.Cu") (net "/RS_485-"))
 (segment (start 142.5 72.5) (end 153 72.5) (width 0.6) (layer "F.Cu") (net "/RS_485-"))
 (segment (start 142.58 65.5) (end 142.58 70.58) (width 0.6) (layer "F.Cu") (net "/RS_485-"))
 (segment (start 169.5 72.5) (end 176.38 72.5) (width 0.6) (layer "F.Cu") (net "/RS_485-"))
 (segment (start 169.58 72.42) (end 169.5 72.5) (width 0.6) (layer "F.Cu") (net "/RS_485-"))
 (segment (start 129.08 70.58) (end 129 70.66) (width 0.6) (layer "F.Cu") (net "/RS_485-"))
 (segment (start 166.5 72.5) (end 169.5 72.5) (width 0.6) (layer "F.Cu") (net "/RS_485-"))
 (segment (start 156.04 72.46) (end 156 72.5) (width 0.6) (layer "F.Cu") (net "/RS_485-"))
 (segment (start 129 72.5) (end 139.5 72.5) (width 0.6) (layer "F.Cu") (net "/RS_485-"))
 (segment (start 153 72.5) (end 156 72.5) (width 0.6) (layer "F.Cu") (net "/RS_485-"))
 (segment (start 156.04 70.58) (end 156.04 72.46) (width 0.6) (layer "F.Cu") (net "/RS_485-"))
 (segment (start 129.08 65.5) (end 129.08 70.58) (width 0.6) (layer "F.Cu") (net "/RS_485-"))
 (segment (start 142.58 70.58) (end 142.58 72.42) (width 0.6) (layer "F.Cu") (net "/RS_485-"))
 (segment (start 169.58 70.58) (end 169.58 72.42) (width 0.6) (layer "F.Cu") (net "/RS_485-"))
 (via (at 139.5 72.5) (size 0.6096) (drill 0.3048) (layers "F.Cu" "B.Cu") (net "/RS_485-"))
 (via (at 166.5 72.5) (size 0.6096) (drill 0.3048) (layers "F.Cu" "B.Cu") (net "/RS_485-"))
 (via (at 126 72.5) (size 0.6096) (drill 0.3048) (layers "F.Cu" "B.Cu") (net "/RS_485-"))
 (via (at 153 72.5) (size 0.6096) (drill 0.3048) (layers "F.Cu" "B.Cu") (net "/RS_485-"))
 (segment (start 126.04 82) (end 126.04 76.92) (width 0.762) (layer "B.Cu") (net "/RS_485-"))
 (segment (start 126 76.88) (end 126.04 76.92) (width 0.762) (layer "B.Cu") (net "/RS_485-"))
 (segment (start 153.04 77) (end 153.04 72.54) (width 0.762) (layer "B.Cu") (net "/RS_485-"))
 (segment (start 153.04 82.08) (end 153.04 77) (width 0.762) (layer "B.Cu") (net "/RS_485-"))
 (segment (start 153.04 72.54) (end 153 72.5) (width 0.762) (layer "B.Cu") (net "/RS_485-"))
 (segment (start 139.46 72.54) (end 139.5 72.5) (width 0.762) (layer "B.Cu") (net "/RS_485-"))
 (segment (start 126 72.5) (end 126 76.88) (width 0.762) (layer "B.Cu") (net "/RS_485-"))
 (segment (start 166.5 77) (end 166.5 72.5) (width 0.762) (layer "B.Cu") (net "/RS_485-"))
 (segment (start 139.46 82) (end 139.46 76.92) (width 0.762) (layer "B.Cu") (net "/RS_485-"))
 (segment (start 139.46 76.92) (end 139.46 72.54) (width 0.762) (layer "B.Cu") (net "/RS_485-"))
 (segment (start 166.5 82.08) (end 166.5 77) (width 0.762) (layer "B.Cu") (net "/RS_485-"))
 (segment (start 131.62 65.5) (end 131.62 63.12) (width 0.762) (layer "F.Cu") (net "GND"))
 (segment (start 158.58 63.08) (end 158.5 63) (width 0.762) (layer "F.Cu") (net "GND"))
 (segment (start 145.12 65.5) (end 145.12 63.12) (width 0.762) (layer "F.Cu") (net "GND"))
 (segment (start 131.5 63) (end 145 63) (width 0.762) (layer "F.Cu") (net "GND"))
 (segment (start 145 63) (end 158.5 63) (width 0.762) (layer "F.Cu") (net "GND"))
 (segment (start 172 65.38) (end 172 63) (width 0.762) (layer "F.Cu") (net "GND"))
 (segment (start 172.12 70.58) (end 172.12 65.5) (width 0.762) (layer "F.Cu") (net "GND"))
 (segment (start 158.58 65.5) (end 158.58 63.08) (width 0.762) (layer "F.Cu") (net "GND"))
 (segment (start 120.5 65) (end 122.5 63) (width 0.762) (layer "F.Cu") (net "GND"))
 (segment (start 120.5 67.5) (end 120.5 65) (width 0.762) (layer "F.Cu") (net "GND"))
 (segment (start 131.62 63.12) (end 131.5 63) (width 0.762) (layer "F.Cu") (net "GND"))
 (segment (start 173.5 63) (end 176.42 65.92) (width 0.762) (layer "F.Cu") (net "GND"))
 (segment (start 122.5 63) (end 131.5 63) (width 0.762) (layer "F.Cu") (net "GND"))
 (segment (start 158.58 70.58) (end 158.58 65.5) (width 0.762) (layer "F.Cu") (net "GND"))
 (segment (start 172.12 65.5) (end 172 65.38) (width 0.762) (layer "F.Cu") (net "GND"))
 (segment (start 131.62 70.58) (end 131.62 65.5) (width 0.762) (layer "F.Cu") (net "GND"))
 (segment (start 111.5 69.96) (end 116.58 69.96) (width 0.762) (layer "F.Cu") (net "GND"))
 (segment (start 158.5 63) (end 172 63) (width 0.762) (layer "F.Cu") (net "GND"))
 (segment (start 145.12 63.12) (end 145 63) (width 0.762) (layer "F.Cu") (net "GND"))
 (segment (start 116.58 69.96) (end 118.04 69.96) (width 0.762) (layer "F.Cu") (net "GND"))
 (segment (start 172 63) (end 173.5 63) (width 0.762) (layer "F.Cu") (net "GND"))
 (segment (start 176.42 65.92) (end 176.42 70) (width 0.762) (layer "F.Cu") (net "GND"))
 (segment (start 118.04 69.96) (end 120.5 67.5) (width 0.762) (layer "F.Cu") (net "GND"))
 (segment (start 176.42 70) (end 181.5 70) (width 0.762) (layer "F.Cu") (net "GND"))
 (segment (start 145.12 70.58) (end 145.12 65.5) (width 0.762) (layer "F.Cu") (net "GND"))
 (segment (start 169.04 84.46) (end 169 84.5) (width 0.762) (layer "B.Cu") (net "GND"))
 (segment (start 155.5 84.5) (end 142 84.5) (width 0.762) (layer "B.Cu") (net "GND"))
 (segment (start 169.04 77) (end 169.04 82.08) (width 0.762) (layer "B.Cu") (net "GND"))
 (segment (start 155.58 77) (end 155.58 82.08) (width 0.762) (layer "B.Cu") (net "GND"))
 (segment (start 155.58 82.08) (end 155.58 84.42) (width 0.762) (layer "B.Cu") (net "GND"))
 (segment (start 169 84.5) (end 155.5 84.5) (width 0.762) (layer "B.Cu") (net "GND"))
 (segment (start 142 82) (end 142 84.5) (width 0.762) (layer "B.Cu") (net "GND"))
 (segment (start 169.04 82.08) (end 169.04 84.46) (width 0.762) (layer "B.Cu") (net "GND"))
 (segment (start 131.08 84.5) (end 128.58 82) (width 0.762) (layer "B.Cu") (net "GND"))
 (segment (start 175.5 70) (end 174.5 71) (width 0.762) (layer "B.Cu") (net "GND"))
 (segment (start 171 84.5) (end 169 84.5) (width 0.762) (layer "B.Cu") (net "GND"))
 (segment (start 142 84.5) (end 131.08 84.5) (width 0.762) (layer "B.Cu") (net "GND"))
 (segment (start 174.5 81) (end 171 84.5) (width 0.762) (layer "B.Cu") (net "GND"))
 (segment (start 128.58 76.92) (end 128.58 82) (width 0.762) (layer "B.Cu") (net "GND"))
 (segment (start 142 76.92) (end 142 82) (width 0.762) (layer "B.Cu") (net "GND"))
 (segment (start 176.42 70) (end 175.5 70) (width 0.762) (layer "B.Cu") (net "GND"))
 (segment (start 155.58 84.42) (end 155.5 84.5) (width 0.762) (layer "B.Cu") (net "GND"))
 (segment (start 174.5 71) (end 174.5 81) (width 0.762) (layer "B.Cu") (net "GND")))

